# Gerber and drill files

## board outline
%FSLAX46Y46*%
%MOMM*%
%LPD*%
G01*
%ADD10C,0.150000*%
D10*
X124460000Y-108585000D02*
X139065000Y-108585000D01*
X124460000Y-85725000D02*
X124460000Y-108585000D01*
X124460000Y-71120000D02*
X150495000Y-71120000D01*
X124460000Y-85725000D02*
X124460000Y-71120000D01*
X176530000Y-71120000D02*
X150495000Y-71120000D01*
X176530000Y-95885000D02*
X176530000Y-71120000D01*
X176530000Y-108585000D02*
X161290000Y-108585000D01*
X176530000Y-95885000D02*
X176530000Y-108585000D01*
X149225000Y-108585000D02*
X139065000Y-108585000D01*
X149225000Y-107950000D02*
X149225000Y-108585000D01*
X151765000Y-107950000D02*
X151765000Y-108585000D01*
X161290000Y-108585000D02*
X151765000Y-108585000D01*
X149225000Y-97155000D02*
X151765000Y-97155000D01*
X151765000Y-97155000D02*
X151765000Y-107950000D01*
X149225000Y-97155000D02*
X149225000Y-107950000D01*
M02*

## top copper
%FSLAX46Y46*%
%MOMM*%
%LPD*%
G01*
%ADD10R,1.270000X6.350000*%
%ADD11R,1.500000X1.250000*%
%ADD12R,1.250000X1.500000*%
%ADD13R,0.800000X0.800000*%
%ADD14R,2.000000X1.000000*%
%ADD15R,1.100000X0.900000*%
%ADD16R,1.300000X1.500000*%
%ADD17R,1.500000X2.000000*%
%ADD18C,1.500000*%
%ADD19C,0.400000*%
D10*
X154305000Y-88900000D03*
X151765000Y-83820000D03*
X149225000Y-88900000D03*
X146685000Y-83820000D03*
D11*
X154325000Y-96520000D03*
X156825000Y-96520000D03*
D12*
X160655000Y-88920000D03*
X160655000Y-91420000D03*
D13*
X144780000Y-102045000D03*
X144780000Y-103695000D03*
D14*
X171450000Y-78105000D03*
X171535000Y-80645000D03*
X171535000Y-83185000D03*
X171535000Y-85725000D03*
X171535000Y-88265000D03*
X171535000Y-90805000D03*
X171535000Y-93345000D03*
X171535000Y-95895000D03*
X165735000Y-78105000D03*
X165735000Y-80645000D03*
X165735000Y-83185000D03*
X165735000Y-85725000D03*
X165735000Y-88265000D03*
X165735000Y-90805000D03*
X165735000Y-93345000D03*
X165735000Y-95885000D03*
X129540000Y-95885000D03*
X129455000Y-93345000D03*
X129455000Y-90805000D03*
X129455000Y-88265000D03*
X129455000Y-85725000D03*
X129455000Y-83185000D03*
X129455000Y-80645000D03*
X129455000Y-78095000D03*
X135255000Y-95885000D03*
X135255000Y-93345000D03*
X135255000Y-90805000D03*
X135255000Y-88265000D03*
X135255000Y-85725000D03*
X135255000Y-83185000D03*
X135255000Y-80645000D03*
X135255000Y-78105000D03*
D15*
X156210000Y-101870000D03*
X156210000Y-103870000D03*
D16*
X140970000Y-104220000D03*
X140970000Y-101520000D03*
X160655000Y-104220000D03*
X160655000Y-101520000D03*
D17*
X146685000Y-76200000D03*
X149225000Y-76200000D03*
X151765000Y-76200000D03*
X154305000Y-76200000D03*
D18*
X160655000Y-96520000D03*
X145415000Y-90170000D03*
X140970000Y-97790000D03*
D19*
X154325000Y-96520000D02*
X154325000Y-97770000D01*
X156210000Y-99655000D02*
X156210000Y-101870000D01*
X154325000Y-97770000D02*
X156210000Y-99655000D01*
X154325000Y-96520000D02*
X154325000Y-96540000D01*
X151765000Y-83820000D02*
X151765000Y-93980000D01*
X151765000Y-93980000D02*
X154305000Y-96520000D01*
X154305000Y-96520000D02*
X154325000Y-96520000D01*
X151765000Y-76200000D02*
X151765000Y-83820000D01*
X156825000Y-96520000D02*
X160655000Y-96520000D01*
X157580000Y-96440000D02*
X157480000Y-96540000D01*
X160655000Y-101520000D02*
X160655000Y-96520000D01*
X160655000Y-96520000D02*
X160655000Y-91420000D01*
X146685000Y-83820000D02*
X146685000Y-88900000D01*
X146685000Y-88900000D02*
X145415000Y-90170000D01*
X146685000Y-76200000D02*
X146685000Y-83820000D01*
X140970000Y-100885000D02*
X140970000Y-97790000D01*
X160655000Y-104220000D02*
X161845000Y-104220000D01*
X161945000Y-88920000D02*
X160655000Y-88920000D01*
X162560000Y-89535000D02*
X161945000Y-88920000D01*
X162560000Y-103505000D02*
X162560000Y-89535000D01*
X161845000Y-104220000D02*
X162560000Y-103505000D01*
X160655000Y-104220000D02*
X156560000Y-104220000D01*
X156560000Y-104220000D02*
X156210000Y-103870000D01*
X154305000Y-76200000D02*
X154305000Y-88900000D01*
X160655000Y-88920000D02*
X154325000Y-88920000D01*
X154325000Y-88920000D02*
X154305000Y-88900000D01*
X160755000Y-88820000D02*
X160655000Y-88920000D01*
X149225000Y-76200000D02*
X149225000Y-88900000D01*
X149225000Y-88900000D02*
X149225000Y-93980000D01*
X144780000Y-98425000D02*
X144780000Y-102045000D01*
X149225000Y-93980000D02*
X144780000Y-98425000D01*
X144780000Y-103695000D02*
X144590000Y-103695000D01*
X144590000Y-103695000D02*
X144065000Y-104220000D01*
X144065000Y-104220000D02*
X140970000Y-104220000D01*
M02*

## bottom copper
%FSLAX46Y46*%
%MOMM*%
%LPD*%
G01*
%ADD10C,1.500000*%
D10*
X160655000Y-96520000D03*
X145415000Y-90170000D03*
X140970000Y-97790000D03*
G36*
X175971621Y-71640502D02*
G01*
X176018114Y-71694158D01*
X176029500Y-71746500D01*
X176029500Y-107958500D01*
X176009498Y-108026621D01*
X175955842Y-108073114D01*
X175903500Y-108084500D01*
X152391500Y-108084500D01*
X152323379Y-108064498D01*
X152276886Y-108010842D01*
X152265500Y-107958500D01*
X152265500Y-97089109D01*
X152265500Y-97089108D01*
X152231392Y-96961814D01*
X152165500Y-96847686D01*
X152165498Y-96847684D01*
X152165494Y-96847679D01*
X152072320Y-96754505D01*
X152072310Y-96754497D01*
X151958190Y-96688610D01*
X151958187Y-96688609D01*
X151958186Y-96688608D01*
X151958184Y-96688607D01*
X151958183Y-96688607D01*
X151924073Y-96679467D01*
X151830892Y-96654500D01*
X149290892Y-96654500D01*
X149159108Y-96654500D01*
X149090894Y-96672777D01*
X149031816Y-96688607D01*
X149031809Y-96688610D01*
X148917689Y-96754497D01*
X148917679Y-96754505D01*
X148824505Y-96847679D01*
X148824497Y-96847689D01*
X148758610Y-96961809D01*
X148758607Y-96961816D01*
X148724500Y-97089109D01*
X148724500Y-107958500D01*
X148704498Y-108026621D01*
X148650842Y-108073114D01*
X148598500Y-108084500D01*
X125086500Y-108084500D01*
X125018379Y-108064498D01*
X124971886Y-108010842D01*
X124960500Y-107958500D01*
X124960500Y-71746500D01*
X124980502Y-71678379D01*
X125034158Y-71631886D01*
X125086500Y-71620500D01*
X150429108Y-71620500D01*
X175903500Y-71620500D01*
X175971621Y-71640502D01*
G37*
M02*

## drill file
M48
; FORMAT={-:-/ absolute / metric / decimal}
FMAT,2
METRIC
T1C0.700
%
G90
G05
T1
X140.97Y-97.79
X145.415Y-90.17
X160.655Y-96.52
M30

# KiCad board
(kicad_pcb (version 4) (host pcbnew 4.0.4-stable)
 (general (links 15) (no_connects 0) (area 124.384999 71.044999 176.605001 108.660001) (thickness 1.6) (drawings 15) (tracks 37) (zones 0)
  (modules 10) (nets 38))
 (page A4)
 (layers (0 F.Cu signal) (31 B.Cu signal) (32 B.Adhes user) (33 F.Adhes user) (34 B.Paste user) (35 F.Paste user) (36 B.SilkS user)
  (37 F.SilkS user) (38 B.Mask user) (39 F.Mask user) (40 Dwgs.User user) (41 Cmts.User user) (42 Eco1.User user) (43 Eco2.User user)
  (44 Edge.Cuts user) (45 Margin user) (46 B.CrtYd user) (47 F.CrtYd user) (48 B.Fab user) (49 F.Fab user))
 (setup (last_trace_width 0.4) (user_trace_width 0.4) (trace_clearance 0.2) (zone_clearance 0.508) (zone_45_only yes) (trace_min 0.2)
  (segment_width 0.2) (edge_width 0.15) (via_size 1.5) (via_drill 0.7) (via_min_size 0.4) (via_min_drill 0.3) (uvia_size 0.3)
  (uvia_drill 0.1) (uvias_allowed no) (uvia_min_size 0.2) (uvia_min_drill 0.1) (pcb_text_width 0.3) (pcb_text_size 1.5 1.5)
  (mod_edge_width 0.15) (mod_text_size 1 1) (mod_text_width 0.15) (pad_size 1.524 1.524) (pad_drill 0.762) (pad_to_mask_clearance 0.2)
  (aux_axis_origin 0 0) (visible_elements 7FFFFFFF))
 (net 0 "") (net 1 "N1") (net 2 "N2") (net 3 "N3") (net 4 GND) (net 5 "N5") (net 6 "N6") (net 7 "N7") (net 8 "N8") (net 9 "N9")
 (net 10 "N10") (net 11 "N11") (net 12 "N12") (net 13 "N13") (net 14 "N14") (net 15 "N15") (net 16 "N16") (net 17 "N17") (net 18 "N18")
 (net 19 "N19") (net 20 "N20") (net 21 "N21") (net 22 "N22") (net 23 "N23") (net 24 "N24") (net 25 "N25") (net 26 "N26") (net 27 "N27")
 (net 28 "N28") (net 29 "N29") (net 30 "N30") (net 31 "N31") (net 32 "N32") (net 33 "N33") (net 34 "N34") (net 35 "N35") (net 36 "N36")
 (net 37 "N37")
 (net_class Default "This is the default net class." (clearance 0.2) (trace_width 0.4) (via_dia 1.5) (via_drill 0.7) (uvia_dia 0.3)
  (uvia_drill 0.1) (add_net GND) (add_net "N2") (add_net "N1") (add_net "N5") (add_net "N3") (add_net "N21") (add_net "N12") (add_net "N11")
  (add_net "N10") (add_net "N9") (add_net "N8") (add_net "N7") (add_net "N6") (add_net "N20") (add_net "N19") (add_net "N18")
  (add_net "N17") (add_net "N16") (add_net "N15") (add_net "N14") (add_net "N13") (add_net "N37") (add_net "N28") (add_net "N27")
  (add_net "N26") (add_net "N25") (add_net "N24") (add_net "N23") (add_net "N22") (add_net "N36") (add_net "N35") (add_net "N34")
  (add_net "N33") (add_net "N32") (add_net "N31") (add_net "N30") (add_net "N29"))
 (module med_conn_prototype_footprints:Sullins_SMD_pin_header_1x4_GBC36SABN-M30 (layer F.Cu) (at 150.495 78.74)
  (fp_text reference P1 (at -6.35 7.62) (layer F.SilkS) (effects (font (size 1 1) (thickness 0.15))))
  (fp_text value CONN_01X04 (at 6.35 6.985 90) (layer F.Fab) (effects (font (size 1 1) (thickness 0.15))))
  (pad 4 smd rect (at 3.81 10.16) (size 1.27 6.35) (layers F.Cu F.Paste F.Mask) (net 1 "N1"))
  (pad 3 smd rect (at 1.27 5.08) (size 1.27 6.35) (layers F.Cu F.Paste F.Mask) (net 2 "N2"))
  (pad 2 smd rect (at -1.27 10.16) (size 1.27 6.35) (layers F.Cu F.Paste F.Mask) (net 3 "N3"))
  (pad 1 smd rect (at -3.81 5.08) (size 1.27 6.35) (layers F.Cu F.Paste F.Mask) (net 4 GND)))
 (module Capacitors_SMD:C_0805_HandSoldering (layer F.Cu) (at 155.575 96.52)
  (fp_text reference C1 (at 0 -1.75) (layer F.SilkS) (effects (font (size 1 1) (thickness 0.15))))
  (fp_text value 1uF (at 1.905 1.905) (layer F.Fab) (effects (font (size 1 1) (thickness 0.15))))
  (pad 1 smd rect (at -1.25 0) (size 1.5 1.25) (layers F.Cu F.Paste F.Mask) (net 2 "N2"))
  (pad 2 smd rect (at 1.25 0) (size 1.5 1.25) (layers F.Cu F.Paste F.Mask) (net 4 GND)))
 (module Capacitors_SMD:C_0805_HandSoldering (layer F.Cu) (at 160.655 90.17 270)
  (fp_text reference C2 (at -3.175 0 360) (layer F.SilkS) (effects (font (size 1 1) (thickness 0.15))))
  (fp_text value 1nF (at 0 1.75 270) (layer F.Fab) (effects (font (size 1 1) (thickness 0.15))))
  (pad 1 smd rect (at -1.25 0 270) (size 1.5 1.25) (layers F.Cu F.Paste F.Mask) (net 1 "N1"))
  (pad 2 smd rect (at 1.25 0 270) (size 1.5 1.25) (layers F.Cu F.Paste F.Mask) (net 4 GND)))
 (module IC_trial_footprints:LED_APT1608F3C (layer F.Cu) (at 144.78 102.87 270)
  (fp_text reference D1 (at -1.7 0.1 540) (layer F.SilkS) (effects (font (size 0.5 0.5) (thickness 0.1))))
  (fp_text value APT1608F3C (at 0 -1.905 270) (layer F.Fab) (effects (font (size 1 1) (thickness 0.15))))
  (pad 2 smd rect (at -0.825 0 270) (size 0.8 0.8) (layers F.Cu F.Paste F.Mask) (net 3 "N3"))
  (pad 1 smd rect (at 0.825 0 270) (size 0.8 0.8) (layers F.Cu F.Paste F.Mask) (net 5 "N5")))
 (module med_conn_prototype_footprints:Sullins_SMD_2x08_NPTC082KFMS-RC (layer F.Cu) (at 161.925 86.995 90)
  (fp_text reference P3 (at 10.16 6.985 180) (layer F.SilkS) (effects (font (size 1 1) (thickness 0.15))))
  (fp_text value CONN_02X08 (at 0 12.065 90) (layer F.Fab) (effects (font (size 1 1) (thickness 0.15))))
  (pad 16 smd rect (at 8.89 9.525 90) (size 1 2) (layers F.Cu F.Paste F.Mask) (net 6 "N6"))
  (pad 15 smd rect (at 6.35 9.61 90) (size 1 2) (layers F.Cu F.Paste F.Mask) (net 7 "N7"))
  (pad 14 smd rect (at 3.81 9.61 90) (size 1 2) (layers F.Cu F.Paste F.Mask) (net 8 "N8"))
  (pad 13 smd rect (at 1.27 9.61 90) (size 1 2) (layers F.Cu F.Paste F.Mask) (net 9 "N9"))
  (pad 12 smd rect (at -1.27 9.61 90) (size 1 2) (layers F.Cu F.Paste F.Mask) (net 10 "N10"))
  (pad 11 smd rect (at -3.81 9.61 90) (size 1 2) (layers F.Cu F.Paste F.Mask) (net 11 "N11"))
  (pad 10 smd rect (at -6.35 9.61 90) (size 1 2) (layers F.Cu F.Paste F.Mask) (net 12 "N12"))
  (pad 9 smd rect (at -8.9 9.61 90) (size 1 2) (layers F.Cu F.Paste F.Mask) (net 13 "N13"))
  (pad 8 smd rect (at 8.89 3.81 90) (size 1 2) (layers F.Cu F.Paste F.Mask) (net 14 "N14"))
  (pad 7 smd rect (at 6.35 3.81 90) (size 1 2) (layers F.Cu F.Paste F.Mask) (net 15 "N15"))
  (pad 6 smd rect (at 3.81 3.81 90) (size 1 2) (layers F.Cu F.Paste F.Mask) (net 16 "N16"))
  (pad 5 smd rect (at 1.27 3.81 90) (size 1 2) (layers F.Cu F.Paste F.Mask) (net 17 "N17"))
  (pad 4 smd rect (at -1.27 3.81 90) (size 1 2) (layers F.Cu F.Paste F.Mask) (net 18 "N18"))
  (pad 3 smd rect (at -3.81 3.81 90) (size 1 2) (layers F.Cu F.Paste F.Mask) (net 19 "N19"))
  (pad 2 smd rect (at -6.35 3.81 90) (size 1 2) (layers F.Cu F.Paste F.Mask) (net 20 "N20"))
  (pad 1 smd rect (at -8.89 3.81 90) (size 1 2) (layers F.Cu F.Paste F.Mask) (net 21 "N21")))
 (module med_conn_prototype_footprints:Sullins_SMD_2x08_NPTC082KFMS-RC (layer F.Cu) (at 139.065 86.995 270)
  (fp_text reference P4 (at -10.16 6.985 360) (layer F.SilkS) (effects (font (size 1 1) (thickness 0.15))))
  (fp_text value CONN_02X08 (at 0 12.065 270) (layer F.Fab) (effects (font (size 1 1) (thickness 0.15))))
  (pad 16 smd rect (at 8.89 9.525 270) (size 1 2) (layers F.Cu F.Paste F.Mask) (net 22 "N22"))
  (pad 15 smd rect (at 6.35 9.61 270) (size 1 2) (layers F.Cu F.Paste F.Mask) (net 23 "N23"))
  (pad 14 smd rect (at 3.81 9.61 270) (size 1 2) (layers F.Cu F.Paste F.Mask) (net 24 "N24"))
  (pad 13 smd rect (at 1.27 9.61 270) (size 1 2) (layers F.Cu F.Paste F.Mask) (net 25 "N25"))
  (pad 12 smd rect (at -1.27 9.61 270) (size 1 2) (layers F.Cu F.Paste F.Mask) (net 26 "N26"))
  (pad 11 smd rect (at -3.81 9.61 270) (size 1 2) (layers F.Cu F.Paste F.Mask) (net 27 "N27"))
  (pad 10 smd rect (at -6.35 9.61 270) (size 1 2) (layers F.Cu F.Paste F.Mask) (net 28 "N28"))
  (pad 9 smd rect (at -8.9 9.61 270) (size 1 2) (layers F.Cu F.Paste F.Mask) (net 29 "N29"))
  (pad 8 smd rect (at 8.89 3.81 270) (size 1 2) (layers F.Cu F.Paste F.Mask) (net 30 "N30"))
  (pad 7 smd rect (at 6.35 3.81 270) (size 1 2) (layers F.Cu F.Paste F.Mask) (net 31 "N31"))
  (pad 6 smd rect (at 3.81 3.81 270) (size 1 2) (layers F.Cu F.Paste F.Mask) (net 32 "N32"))
  (pad 5 smd rect (at 1.27 3.81 270) (size 1 2) (layers F.Cu F.Paste F.Mask) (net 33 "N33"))
  (pad 4 smd rect (at -1.27 3.81 270) (size 1 2) (layers F.Cu F.Paste F.Mask) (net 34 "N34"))
  (pad 3 smd rect (at -3.81 3.81 270) (size 1 2) (layers F.Cu F.Paste F.Mask) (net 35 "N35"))
  (pad 2 smd rect (at -6.35 3.81 270) (size 1 2) (layers F.Cu F.Paste F.Mask) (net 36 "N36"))
  (pad 1 smd rect (at -8.89 3.81 270) (size 1 2) (layers F.Cu F.Paste F.Mask) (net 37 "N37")))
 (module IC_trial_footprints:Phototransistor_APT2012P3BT (layer F.Cu) (at 156.21 102.87 90)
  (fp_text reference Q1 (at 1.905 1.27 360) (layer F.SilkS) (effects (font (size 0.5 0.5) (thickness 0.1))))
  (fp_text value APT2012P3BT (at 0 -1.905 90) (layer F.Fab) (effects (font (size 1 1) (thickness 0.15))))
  (pad 2 smd rect (at 1 0 90) (size 0.9 1.1) (layers F.Cu F.Paste F.Mask) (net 2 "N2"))
  (pad 1 smd rect (at -1 0 90) (size 0.9 1.1) (layers F.Cu F.Paste F.Mask) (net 1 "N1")))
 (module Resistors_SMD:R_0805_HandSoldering (layer F.Cu) (at 140.97 102.87 90)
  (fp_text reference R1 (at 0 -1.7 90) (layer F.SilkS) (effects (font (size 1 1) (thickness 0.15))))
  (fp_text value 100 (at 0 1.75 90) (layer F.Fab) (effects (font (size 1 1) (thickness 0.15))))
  (pad 1 smd rect (at -1.35 0 90) (size 1.5 1.3) (layers F.Cu F.Paste F.Mask) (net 5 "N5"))
  (pad 2 smd rect (at 1.35 0 90) (size 1.5 1.3) (layers F.Cu F.Paste F.Mask) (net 4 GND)))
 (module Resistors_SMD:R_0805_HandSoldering (layer F.Cu) (at 160.655 102.87 90)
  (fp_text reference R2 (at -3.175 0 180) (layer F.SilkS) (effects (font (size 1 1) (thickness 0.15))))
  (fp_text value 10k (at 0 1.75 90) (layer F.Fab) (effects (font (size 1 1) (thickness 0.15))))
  (pad 1 smd rect (at -1.35 0 90) (size 1.5 1.3) (layers F.Cu F.Paste F.Mask) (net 1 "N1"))
  (pad 2 smd rect (at 1.35 0 90) (size 1.5 1.3) (layers F.Cu F.Paste F.Mask) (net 4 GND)))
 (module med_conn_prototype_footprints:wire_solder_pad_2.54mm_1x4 (layer F.Cu) (at 150.495 72.39)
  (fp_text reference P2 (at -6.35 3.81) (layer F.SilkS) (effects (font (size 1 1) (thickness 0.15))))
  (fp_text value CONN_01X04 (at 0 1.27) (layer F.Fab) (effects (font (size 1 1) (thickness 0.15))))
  (pad 1 smd rect (at -3.81 3.81) (size 1.5 2) (layers F.Cu F.Paste F.Mask) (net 4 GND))
  (pad 2 smd rect (at -1.27 3.81) (size 1.5 2) (layers F.Cu F.Paste F.Mask) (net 3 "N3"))
  (pad 3 smd rect (at 1.27 3.81) (size 1.5 2) (layers F.Cu F.Paste F.Mask) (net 2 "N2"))
  (pad 4 smd rect (at 3.81 3.81) (size 1.5 2) (layers F.Cu F.Paste F.Mask) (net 1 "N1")))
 (gr_line (start 124.46 108.585) (end 139.065 108.585) (angle 90) (layer Edge.Cuts) (width 0.15))
 (gr_line (start 124.46 85.725) (end 124.46 108.585) (angle 90) (layer Edge.Cuts) (width 0.15))
 (gr_line (start 124.46 71.12) (end 150.495 71.12) (angle 90) (layer Edge.Cuts) (width 0.15))
 (gr_line (start 124.46 85.725) (end 124.46 71.12) (angle 90) (layer Edge.Cuts) (width 0.15))
 (gr_line (start 176.53 71.12) (end 150.495 71.12) (angle 90) (layer Edge.Cuts) (width 0.15))
 (gr_line (start 176.53 95.885) (end 176.53 71.12) (angle 90) (layer Edge.Cuts) (width 0.15))
 (gr_line (start 176.53 108.585) (end 161.29 108.585) (angle 90) (layer Edge.Cuts) (width 0.15))
 (gr_line (start 176.53 95.885) (end 176.53 108.585) (angle 90) (layer Edge.Cuts) (width 0.15))
 (gr_line (start 149.225 108.585) (end 139.065 108.585) (angle 90) (layer Edge.Cuts) (width 0.15))
 (gr_line (start 149.225 107.95) (end 149.225 108.585) (angle 90) (layer Edge.Cuts) (width 0.15))
 (gr_line (start 151.765 107.95) (end 151.765 108.585) (angle 90) (layer Edge.Cuts) (width 0.15))
 (gr_line (start 161.29 108.585) (end 151.765 108.585) (angle 90) (layer Edge.Cuts) (width 0.15))
 (gr_line (start 149.225 97.155) (end 151.765 97.155) (angle 90) (layer Edge.Cuts) (width 0.15))
 (gr_line (start 151.765 97.155) (end 151.765 107.95) (angle 90) (layer Edge.Cuts) (width 0.15))
 (gr_line (start 149.225 97.155) (end 149.225 107.95) (angle 90) (layer Edge.Cuts) (width 0.15))
 (segment (start 154.325 96.52) (end 154.325 97.77) (width 0.4) (layer F.Cu) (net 2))
 (segment (start 156.21 99.655) (end 156.21 101.87) (width 0.4) (layer F.Cu) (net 2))
 (segment (start 154.325 97.77) (end 156.21 99.655) (width 0.4) (layer F.Cu) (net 2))
 (segment (start 154.325 96.52) (end 154.325 96.54) (width 0.4) (layer F.Cu) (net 2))
 (segment (start 151.765 83.82) (end 151.765 93.98) (width 0.4) (layer F.Cu) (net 2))
 (segment (start 151.765 93.98) (end 154.305 96.52) (width 0.4) (layer F.Cu) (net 2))
 (segment (start 154.305 96.52) (end 154.325 96.52) (width 0.4) (layer F.Cu) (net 2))
 (segment (start 151.765 76.2) (end 151.765 83.82) (width 0.4) (layer F.Cu) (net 2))
 (segment (start 156.825 96.52) (end 160.655 96.52) (width 0.4) (layer F.Cu) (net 4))
 (via (at 160.655 96.52) (size 1.5) (drill 0.7) (layers F.Cu B.Cu) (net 4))
 (segment (start 157.58 96.44) (end 157.48 96.54) (width 0.4) (layer F.Cu) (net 4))
 (segment (start 160.655 101.52) (end 160.655 96.52) (width 0.4) (layer F.Cu) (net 4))
 (segment (start 160.655 96.52) (end 160.655 91.42) (width 0.4) (layer F.Cu) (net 4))
 (segment (start 146.685 83.82) (end 146.685 88.9) (width 0.4) (layer F.Cu) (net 4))
 (via (at 145.415 90.17) (size 1.5) (drill 0.7) (layers F.Cu B.Cu) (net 4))
 (segment (start 146.685 88.9) (end 145.415 90.17) (width 0.4) (layer F.Cu) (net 4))
 (segment (start 146.685 76.2) (end 146.685 83.82) (width 0.4) (layer F.Cu) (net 4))
 (segment (start 140.97 100.885) (end 140.97 97.79) (width 0.4) (layer F.Cu) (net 4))
 (via (at 140.97 97.79) (size 1.5) (drill 0.7) (layers F.Cu B.Cu) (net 4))
 (segment (start 160.655 104.22) (end 161.845 104.22) (width 0.4) (layer F.Cu) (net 1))
 (segment (start 161.945 88.92) (end 160.655 88.92) (width 0.4) (layer F.Cu) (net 1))
 (segment (start 162.56 89.535) (end 161.945 88.92) (width 0.4) (layer F.Cu) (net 1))
 (segment (start 162.56 103.505) (end 162.56 89.535) (width 0.4) (layer F.Cu) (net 1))
 (segment (start 161.845 104.22) (end 162.56 103.505) (width 0.4) (layer F.Cu) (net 1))
 (segment (start 160.655 104.22) (end 156.56 104.22) (width 0.4) (layer F.Cu) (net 1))
 (segment (start 156.56 104.22) (end 156.21 103.87) (width 0.4) (layer F.Cu) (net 1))
 (segment (start 154.305 76.2) (end 154.305 88.9) (width 0.4) (layer F.Cu) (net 1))
 (segment (start 160.655 88.92) (end 154.325 88.92) (width 0.4) (layer F.Cu) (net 1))
 (segment (start 154.325 88.92) (end 154.305 88.9) (width 0.4) (layer F.Cu) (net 1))
 (segment (start 160.755 88.82) (end 160.655 88.92) (width 0.4) (layer F.Cu) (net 1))
 (segment (start 149.225 76.2) (end 149.225 88.9) (width 0.4) (layer F.Cu) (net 3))
 (segment (start 149.225 88.9) (end 149.225 93.98) (width 0.4) (layer F.Cu) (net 3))
 (segment (start 144.78 98.425) (end 144.78 102.045) (width 0.4) (layer F.Cu) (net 3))
 (segment (start 149.225 93.98) (end 144.78 98.425) (width 0.4) (layer F.Cu) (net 3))
 (segment (start 144.78 103.695) (end 144.59 103.695) (width 0.4) (layer F.Cu) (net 5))
 (segment (start 144.59 103.695) (end 144.065 104.22) (width 0.4) (layer F.Cu) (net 5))
 (segment (start 144.065 104.22) (end 140.97 104.22) (width 0.4) (layer F.Cu) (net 5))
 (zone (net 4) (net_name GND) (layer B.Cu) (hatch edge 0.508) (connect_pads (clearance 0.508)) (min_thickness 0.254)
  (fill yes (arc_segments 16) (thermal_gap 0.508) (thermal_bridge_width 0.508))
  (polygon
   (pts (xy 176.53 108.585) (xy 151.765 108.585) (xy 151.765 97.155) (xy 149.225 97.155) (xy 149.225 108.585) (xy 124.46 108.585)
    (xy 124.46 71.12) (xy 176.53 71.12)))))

